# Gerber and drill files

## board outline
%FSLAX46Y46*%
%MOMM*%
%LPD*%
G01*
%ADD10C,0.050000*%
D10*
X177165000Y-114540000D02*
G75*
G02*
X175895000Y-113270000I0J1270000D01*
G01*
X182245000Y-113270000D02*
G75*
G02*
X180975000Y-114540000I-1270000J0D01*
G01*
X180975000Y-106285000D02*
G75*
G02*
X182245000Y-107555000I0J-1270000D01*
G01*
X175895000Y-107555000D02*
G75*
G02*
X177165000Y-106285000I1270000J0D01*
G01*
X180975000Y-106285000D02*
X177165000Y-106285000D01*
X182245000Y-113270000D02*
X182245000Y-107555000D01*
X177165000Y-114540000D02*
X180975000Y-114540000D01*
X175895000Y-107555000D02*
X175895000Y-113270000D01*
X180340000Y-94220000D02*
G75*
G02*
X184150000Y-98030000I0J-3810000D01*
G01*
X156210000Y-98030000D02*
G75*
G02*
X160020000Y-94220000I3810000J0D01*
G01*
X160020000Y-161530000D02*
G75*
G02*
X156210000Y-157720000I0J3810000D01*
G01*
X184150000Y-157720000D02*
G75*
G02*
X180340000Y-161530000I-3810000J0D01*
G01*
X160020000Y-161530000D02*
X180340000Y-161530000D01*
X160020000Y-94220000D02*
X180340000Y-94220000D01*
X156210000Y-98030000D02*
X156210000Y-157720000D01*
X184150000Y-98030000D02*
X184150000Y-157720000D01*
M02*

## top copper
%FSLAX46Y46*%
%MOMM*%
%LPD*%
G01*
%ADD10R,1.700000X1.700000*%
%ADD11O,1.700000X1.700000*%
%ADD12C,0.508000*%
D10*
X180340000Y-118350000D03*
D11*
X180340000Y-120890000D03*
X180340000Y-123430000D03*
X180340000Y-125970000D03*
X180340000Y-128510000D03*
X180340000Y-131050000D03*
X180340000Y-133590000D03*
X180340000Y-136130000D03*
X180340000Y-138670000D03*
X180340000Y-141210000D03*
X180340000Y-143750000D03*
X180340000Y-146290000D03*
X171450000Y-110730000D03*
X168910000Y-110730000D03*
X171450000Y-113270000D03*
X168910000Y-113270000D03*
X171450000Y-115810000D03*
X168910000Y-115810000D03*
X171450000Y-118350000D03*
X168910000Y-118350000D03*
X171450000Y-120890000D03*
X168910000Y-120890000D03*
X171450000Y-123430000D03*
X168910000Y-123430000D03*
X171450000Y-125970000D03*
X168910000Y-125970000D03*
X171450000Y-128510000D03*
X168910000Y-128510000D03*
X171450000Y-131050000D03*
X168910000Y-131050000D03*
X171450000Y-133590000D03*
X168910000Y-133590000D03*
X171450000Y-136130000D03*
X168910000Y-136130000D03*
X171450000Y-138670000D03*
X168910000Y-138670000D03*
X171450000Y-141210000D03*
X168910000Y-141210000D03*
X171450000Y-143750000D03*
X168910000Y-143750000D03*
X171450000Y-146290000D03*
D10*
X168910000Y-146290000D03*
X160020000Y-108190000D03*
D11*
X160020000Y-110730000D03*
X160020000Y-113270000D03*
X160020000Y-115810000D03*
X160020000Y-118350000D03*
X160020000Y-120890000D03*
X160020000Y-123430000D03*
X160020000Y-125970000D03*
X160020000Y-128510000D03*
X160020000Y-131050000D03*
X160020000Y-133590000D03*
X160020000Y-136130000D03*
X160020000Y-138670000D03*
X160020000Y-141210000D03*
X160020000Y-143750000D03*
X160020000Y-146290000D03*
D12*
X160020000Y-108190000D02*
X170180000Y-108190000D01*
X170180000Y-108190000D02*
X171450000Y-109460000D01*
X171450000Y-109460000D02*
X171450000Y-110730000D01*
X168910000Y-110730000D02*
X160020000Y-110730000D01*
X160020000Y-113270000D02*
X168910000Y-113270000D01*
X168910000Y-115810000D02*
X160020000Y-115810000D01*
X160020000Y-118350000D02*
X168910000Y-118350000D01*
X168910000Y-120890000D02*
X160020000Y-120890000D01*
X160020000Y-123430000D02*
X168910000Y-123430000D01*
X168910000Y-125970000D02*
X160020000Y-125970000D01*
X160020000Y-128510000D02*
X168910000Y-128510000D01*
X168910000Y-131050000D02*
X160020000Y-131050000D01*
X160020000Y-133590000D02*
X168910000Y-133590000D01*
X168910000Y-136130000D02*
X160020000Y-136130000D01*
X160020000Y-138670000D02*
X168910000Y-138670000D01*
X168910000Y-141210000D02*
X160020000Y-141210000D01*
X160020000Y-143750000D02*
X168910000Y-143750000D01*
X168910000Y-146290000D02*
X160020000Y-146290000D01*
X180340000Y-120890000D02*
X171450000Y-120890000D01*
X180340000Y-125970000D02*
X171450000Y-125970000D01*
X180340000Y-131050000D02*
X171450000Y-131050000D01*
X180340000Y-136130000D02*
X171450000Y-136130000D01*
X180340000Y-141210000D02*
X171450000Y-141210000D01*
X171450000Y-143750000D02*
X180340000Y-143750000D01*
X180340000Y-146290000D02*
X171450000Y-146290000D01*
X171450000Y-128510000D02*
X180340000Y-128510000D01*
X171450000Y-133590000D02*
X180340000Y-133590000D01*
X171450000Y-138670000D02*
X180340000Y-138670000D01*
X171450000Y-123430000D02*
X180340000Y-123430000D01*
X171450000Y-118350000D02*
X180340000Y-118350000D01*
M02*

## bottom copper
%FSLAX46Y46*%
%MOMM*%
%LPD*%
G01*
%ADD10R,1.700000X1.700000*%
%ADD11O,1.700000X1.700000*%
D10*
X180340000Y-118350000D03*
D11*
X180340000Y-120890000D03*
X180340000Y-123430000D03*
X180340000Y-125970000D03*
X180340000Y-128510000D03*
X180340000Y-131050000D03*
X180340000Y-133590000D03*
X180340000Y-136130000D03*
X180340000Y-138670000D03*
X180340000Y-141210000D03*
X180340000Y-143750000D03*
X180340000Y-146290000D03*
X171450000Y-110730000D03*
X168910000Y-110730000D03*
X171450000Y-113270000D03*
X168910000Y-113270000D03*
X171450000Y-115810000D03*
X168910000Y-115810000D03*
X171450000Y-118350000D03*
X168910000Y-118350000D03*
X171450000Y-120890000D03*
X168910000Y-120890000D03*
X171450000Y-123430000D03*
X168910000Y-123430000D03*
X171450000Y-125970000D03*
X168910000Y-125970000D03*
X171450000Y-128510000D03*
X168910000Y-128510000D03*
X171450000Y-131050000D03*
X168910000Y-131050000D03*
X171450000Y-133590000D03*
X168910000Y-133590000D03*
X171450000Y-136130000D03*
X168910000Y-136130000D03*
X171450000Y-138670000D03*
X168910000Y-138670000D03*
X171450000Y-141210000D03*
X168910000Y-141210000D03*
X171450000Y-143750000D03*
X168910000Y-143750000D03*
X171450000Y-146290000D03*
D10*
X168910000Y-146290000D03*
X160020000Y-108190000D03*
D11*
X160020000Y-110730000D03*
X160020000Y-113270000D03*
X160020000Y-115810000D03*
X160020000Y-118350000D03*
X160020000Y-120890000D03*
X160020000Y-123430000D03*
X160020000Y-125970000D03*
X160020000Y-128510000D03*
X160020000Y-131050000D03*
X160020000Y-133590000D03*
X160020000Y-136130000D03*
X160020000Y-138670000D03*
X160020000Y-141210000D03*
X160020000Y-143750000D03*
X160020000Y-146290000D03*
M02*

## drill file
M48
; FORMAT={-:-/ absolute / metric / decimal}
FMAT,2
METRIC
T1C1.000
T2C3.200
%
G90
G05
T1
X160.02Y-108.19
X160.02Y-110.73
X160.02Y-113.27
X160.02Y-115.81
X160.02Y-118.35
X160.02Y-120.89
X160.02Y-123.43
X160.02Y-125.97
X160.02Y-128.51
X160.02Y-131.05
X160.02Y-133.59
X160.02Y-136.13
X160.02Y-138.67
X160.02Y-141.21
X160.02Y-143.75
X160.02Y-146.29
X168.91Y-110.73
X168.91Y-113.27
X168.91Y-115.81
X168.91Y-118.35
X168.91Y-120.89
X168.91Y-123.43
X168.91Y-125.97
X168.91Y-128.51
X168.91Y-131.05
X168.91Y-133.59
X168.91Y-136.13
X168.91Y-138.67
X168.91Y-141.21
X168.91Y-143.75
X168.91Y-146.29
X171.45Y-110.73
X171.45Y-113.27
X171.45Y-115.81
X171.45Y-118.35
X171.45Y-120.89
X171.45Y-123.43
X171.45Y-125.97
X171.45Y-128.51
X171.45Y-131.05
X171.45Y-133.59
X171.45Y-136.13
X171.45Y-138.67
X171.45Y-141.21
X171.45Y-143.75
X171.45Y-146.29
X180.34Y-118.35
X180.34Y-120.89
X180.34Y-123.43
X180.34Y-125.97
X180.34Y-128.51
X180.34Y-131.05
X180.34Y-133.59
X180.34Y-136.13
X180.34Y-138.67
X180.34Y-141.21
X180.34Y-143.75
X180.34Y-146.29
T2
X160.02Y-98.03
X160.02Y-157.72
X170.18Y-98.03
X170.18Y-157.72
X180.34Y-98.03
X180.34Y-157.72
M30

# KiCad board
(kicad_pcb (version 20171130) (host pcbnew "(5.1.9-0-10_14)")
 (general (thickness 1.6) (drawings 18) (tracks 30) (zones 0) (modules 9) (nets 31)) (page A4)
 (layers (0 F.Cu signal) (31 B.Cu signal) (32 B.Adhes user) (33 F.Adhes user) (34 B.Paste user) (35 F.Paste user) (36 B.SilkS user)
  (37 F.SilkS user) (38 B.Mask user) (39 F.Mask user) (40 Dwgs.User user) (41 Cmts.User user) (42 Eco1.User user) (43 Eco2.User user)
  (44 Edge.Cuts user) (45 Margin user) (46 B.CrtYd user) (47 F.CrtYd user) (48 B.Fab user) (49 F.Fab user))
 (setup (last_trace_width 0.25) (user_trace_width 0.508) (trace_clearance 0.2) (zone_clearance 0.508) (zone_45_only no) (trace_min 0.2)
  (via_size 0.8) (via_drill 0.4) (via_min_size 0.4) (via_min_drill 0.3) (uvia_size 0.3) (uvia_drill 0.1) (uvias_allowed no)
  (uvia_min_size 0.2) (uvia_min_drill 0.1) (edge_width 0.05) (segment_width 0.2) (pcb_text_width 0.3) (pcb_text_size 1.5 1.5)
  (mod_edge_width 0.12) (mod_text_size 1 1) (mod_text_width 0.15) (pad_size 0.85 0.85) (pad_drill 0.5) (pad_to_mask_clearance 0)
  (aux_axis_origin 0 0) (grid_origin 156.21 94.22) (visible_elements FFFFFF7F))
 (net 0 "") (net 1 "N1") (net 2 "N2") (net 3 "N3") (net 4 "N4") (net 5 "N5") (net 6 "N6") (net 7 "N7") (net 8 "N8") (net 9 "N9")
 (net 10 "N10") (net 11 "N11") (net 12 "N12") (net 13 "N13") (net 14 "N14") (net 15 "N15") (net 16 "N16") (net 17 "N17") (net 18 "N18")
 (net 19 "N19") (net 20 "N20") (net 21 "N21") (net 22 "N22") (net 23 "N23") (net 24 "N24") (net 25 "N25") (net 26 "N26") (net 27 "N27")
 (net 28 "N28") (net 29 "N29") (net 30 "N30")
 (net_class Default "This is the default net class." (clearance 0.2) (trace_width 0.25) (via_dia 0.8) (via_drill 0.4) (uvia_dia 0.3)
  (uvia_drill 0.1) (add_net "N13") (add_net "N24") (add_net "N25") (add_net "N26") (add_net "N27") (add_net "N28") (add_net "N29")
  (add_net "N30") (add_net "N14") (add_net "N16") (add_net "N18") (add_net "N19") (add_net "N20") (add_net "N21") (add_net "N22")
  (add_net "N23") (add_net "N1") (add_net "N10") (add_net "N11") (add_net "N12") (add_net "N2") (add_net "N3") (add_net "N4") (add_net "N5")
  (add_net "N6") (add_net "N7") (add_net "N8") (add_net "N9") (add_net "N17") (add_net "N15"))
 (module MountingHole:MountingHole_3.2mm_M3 (layer F.Cu) (at 170.18 157.72)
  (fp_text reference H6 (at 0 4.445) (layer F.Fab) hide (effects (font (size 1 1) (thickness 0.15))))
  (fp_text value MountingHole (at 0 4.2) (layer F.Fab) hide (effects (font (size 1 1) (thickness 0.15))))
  (pad 1 np_thru_hole circle (at 0 0) (size 3.2 3.2) (drill 3.2) (layers *.Cu *.Mask)))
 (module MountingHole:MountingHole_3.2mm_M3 (layer F.Cu) (at 170.18 98.03)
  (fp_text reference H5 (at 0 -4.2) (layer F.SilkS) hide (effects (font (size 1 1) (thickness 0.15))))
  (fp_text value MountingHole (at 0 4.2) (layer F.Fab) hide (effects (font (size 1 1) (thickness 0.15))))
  (pad 1 np_thru_hole circle (at 0 0) (size 3.2 3.2) (drill 3.2) (layers *.Cu *.Mask)))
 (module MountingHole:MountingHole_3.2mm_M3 (layer F.Cu) (at 180.34 157.72)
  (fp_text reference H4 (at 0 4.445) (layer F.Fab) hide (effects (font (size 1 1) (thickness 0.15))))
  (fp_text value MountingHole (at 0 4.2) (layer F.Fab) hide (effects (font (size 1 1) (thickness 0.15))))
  (pad 1 np_thru_hole circle (at 0 0) (size 3.2 3.2) (drill 3.2) (layers *.Cu *.Mask)))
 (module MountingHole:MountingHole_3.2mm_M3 (layer F.Cu) (at 180.34 98.03)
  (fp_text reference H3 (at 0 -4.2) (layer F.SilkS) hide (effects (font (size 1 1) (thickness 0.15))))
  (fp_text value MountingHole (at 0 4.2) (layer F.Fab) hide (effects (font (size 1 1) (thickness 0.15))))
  (pad 1 np_thru_hole circle (at 0 0) (size 3.2 3.2) (drill 3.2) (layers *.Cu *.Mask)))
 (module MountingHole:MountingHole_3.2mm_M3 (layer F.Cu) (at 160.02 157.72)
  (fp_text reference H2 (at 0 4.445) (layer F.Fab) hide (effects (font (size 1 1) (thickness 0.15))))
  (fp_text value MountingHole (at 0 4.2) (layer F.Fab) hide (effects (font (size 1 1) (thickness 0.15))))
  (pad 1 np_thru_hole circle (at 0 0) (size 3.2 3.2) (drill 3.2) (layers *.Cu *.Mask)))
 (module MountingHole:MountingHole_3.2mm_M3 (layer F.Cu) (at 160.02 98.03)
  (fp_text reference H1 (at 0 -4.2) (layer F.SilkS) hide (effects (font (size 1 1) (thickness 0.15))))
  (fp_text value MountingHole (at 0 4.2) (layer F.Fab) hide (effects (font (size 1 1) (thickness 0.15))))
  (pad 1 np_thru_hole circle (at 0 0) (size 3.2 3.2) (drill 3.2) (layers *.Cu *.Mask)))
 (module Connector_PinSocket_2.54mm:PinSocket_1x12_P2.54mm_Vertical (layer F.Cu) (at 180.34 118.35)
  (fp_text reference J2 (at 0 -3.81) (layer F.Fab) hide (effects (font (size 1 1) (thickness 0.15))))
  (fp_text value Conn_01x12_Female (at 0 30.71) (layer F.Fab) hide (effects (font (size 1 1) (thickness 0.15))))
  (pad 1 thru_hole rect (at 0 0) (size 1.7 1.7) (drill 1) (layers *.Cu *.Mask) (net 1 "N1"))
  (pad 2 thru_hole oval (at 0 2.54) (size 1.7 1.7) (drill 1) (layers *.Cu *.Mask) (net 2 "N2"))
  (pad 3 thru_hole oval (at 0 5.08) (size 1.7 1.7) (drill 1) (layers *.Cu *.Mask) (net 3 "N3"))
  (pad 4 thru_hole oval (at 0 7.62) (size 1.7 1.7) (drill 1) (layers *.Cu *.Mask) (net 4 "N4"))
  (pad 5 thru_hole oval (at 0 10.16) (size 1.7 1.7) (drill 1) (layers *.Cu *.Mask) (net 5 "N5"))
  (pad 6 thru_hole oval (at 0 12.7) (size 1.7 1.7) (drill 1) (layers *.Cu *.Mask) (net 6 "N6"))
  (pad 7 thru_hole oval (at 0 15.24) (size 1.7 1.7) (drill 1) (layers *.Cu *.Mask) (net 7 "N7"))
  (pad 8 thru_hole oval (at 0 17.78) (size 1.7 1.7) (drill 1) (layers *.Cu *.Mask) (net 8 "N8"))
  (pad 9 thru_hole oval (at 0 20.32) (size 1.7 1.7) (drill 1) (layers *.Cu *.Mask) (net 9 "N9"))
  (pad 10 thru_hole oval (at 0 22.86) (size 1.7 1.7) (drill 1) (layers *.Cu *.Mask) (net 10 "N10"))
  (pad 11 thru_hole oval (at 0 25.4) (size 1.7 1.7) (drill 1) (layers *.Cu *.Mask) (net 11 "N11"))
  (pad 12 thru_hole oval (at 0 27.94) (size 1.7 1.7) (drill 1) (layers *.Cu *.Mask) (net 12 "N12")))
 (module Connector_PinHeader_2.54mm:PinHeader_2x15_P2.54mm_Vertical (layer B.Cu) (at 168.91 146.29)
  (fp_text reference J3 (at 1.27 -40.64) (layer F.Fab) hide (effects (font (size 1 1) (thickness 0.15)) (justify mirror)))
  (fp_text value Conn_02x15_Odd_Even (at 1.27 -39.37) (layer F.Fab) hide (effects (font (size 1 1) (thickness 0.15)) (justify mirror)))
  (pad 30 thru_hole oval (at 2.54 -35.56) (size 1.7 1.7) (drill 1) (layers *.Cu *.Mask) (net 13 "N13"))
  (pad 29 thru_hole oval (at 0 -35.56) (size 1.7 1.7) (drill 1) (layers *.Cu *.Mask) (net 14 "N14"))
  (pad 28 thru_hole oval (at 2.54 -33.02) (size 1.7 1.7) (drill 1) (layers *.Cu *.Mask) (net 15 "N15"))
  (pad 27 thru_hole oval (at 0 -33.02) (size 1.7 1.7) (drill 1) (layers *.Cu *.Mask) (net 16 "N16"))
  (pad 26 thru_hole oval (at 2.54 -30.48) (size 1.7 1.7) (drill 1) (layers *.Cu *.Mask) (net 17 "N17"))
  (pad 25 thru_hole oval (at 0 -30.48) (size 1.7 1.7) (drill 1) (layers *.Cu *.Mask) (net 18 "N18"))
  (pad 24 thru_hole oval (at 2.54 -27.94) (size 1.7 1.7) (drill 1) (layers *.Cu *.Mask) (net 1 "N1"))
  (pad 23 thru_hole oval (at 0 -27.94) (size 1.7 1.7) (drill 1) (layers *.Cu *.Mask) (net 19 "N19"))
  (pad 22 thru_hole oval (at 2.54 -25.4) (size 1.7 1.7) (drill 1) (layers *.Cu *.Mask) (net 2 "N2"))
  (pad 21 thru_hole oval (at 0 -25.4) (size 1.7 1.7) (drill 1) (layers *.Cu *.Mask) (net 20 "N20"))
  (pad 20 thru_hole oval (at 2.54 -22.86) (size 1.7 1.7) (drill 1) (layers *.Cu *.Mask) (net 3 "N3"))
  (pad 19 thru_hole oval (at 0 -22.86) (size 1.7 1.7) (drill 1) (layers *.Cu *.Mask) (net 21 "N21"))
  (pad 18 thru_hole oval (at 2.54 -20.32) (size 1.7 1.7) (drill 1) (layers *.Cu *.Mask) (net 4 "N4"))
  (pad 17 thru_hole oval (at 0 -20.32) (size 1.7 1.7) (drill 1) (layers *.Cu *.Mask) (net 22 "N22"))
  (pad 16 thru_hole oval (at 2.54 -17.78) (size 1.7 1.7) (drill 1) (layers *.Cu *.Mask) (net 5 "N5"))
  (pad 15 thru_hole oval (at 0 -17.78) (size 1.7 1.7) (drill 1) (layers *.Cu *.Mask) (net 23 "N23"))
  (pad 14 thru_hole oval (at 2.54 -15.24) (size 1.7 1.7) (drill 1) (layers *.Cu *.Mask) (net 6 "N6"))
  (pad 13 thru_hole oval (at 0 -15.24) (size 1.7 1.7) (drill 1) (layers *.Cu *.Mask) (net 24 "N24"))
  (pad 12 thru_hole oval (at 2.54 -12.7) (size 1.7 1.7) (drill 1) (layers *.Cu *.Mask) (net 7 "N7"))
  (pad 11 thru_hole oval (at 0 -12.7) (size 1.7 1.7) (drill 1) (layers *.Cu *.Mask) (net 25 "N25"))
  (pad 10 thru_hole oval (at 2.54 -10.16) (size 1.7 1.7) (drill 1) (layers *.Cu *.Mask) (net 8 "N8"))
  (pad 9 thru_hole oval (at 0 -10.16) (size 1.7 1.7) (drill 1) (layers *.Cu *.Mask) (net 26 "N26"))
  (pad 8 thru_hole oval (at 2.54 -7.62) (size 1.7 1.7) (drill 1) (layers *.Cu *.Mask) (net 9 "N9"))
  (pad 7 thru_hole oval (at 0 -7.62) (size 1.7 1.7) (drill 1) (layers *.Cu *.Mask) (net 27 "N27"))
  (pad 6 thru_hole oval (at 2.54 -5.08) (size 1.7 1.7) (drill 1) (layers *.Cu *.Mask) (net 10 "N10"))
  (pad 5 thru_hole oval (at 0 -5.08) (size 1.7 1.7) (drill 1) (layers *.Cu *.Mask) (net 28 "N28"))
  (pad 4 thru_hole oval (at 2.54 -2.54) (size 1.7 1.7) (drill 1) (layers *.Cu *.Mask) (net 11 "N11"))
  (pad 3 thru_hole oval (at 0 -2.54) (size 1.7 1.7) (drill 1) (layers *.Cu *.Mask) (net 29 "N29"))
  (pad 2 thru_hole oval (at 2.54 0) (size 1.7 1.7) (drill 1) (layers *.Cu *.Mask) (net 12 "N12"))
  (pad 1 thru_hole rect (at 0 0) (size 1.7 1.7) (drill 1) (layers *.Cu *.Mask) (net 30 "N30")))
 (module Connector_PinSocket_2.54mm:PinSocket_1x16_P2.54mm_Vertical (layer F.Cu) (at 160.02 108.19)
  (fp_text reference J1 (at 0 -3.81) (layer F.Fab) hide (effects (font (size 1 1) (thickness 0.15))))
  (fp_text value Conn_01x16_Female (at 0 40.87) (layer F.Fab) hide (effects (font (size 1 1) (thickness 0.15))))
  (pad 1 thru_hole rect (at 0 0) (size 1.7 1.7) (drill 1) (layers *.Cu *.Mask) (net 13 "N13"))
  (pad 2 thru_hole oval (at 0 2.54) (size 1.7 1.7) (drill 1) (layers *.Cu *.Mask) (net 14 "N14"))
  (pad 3 thru_hole oval (at 0 5.08) (size 1.7 1.7) (drill 1) (layers *.Cu *.Mask) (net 16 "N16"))
  (pad 4 thru_hole oval (at 0 7.62) (size 1.7 1.7) (drill 1) (layers *.Cu *.Mask) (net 18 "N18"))
  (pad 5 thru_hole oval (at 0 10.16) (size 1.7 1.7) (drill 1) (layers *.Cu *.Mask) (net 19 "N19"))
  (pad 6 thru_hole oval (at 0 12.7) (size 1.7 1.7) (drill 1) (layers *.Cu *.Mask) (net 20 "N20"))
  (pad 7 thru_hole oval (at 0 15.24) (size 1.7 1.7) (drill 1) (layers *.Cu *.Mask) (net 21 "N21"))
  (pad 8 thru_hole oval (at 0 17.78) (size 1.7 1.7) (drill 1) (layers *.Cu *.Mask) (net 22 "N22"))
  (pad 9 thru_hole oval (at 0 20.32) (size 1.7 1.7) (drill 1) (layers *.Cu *.Mask) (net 23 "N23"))
  (pad 10 thru_hole oval (at 0 22.86) (size 1.7 1.7) (drill 1) (layers *.Cu *.Mask) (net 24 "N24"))
  (pad 11 thru_hole oval (at 0 25.4) (size 1.7 1.7) (drill 1) (layers *.Cu *.Mask) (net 25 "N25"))
  (pad 12 thru_hole oval (at 0 27.94) (size 1.7 1.7) (drill 1) (layers *.Cu *.Mask) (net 26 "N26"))
  (pad 13 thru_hole oval (at 0 30.48) (size 1.7 1.7) (drill 1) (layers *.Cu *.Mask) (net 27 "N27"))
  (pad 14 thru_hole oval (at 0 33.02) (size 1.7 1.7) (drill 1) (layers *.Cu *.Mask) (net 28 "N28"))
  (pad 15 thru_hole oval (at 0 35.56) (size 1.7 1.7) (drill 1) (layers *.Cu *.Mask) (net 29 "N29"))
  (pad 16 thru_hole oval (at 0 38.1) (size 1.7 1.7) (drill 1) (layers *.Cu *.Mask) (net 30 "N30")))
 (gr_arc (start 177.165 113.27) (end 175.895 113.27) (angle -90) (layer Edge.Cuts) (width 0.05))
 (gr_arc (start 180.975 113.27) (end 180.975 114.54) (angle -90) (layer Edge.Cuts) (width 0.05))
 (gr_arc (start 180.975 107.555) (end 182.245 107.555) (angle -90) (layer Edge.Cuts) (width 0.05))
 (gr_arc (start 177.165 107.555) (end 177.165 106.285) (angle -90) (layer Edge.Cuts) (width 0.05))
 (gr_line (start 180.975 106.285) (end 177.165 106.285) (layer Edge.Cuts) (width 0.05))
 (gr_line (start 182.245 113.27) (end 182.245 107.555) (layer Edge.Cuts) (width 0.05))
 (gr_line (start 177.165 114.54) (end 180.975 114.54) (layer Edge.Cuts) (width 0.05))
 (gr_line (start 175.895 107.555) (end 175.895 113.27) (layer Edge.Cuts) (width 0.05))
 (gr_arc (start 180.34 98.03) (end 184.15 98.03) (angle -90) (layer Edge.Cuts) (width 0.05))
 (gr_arc (start 160.02 98.03) (end 160.02 94.22) (angle -90) (layer Edge.Cuts) (width 0.05))
 (gr_arc (start 160.02 157.72) (end 156.21 157.72) (angle -90) (layer Edge.Cuts) (width 0.05))
 (gr_arc (start 180.34 157.72) (end 180.34 161.53) (angle -90) (layer Edge.Cuts) (width 0.05))
 (gr_line (start 160.02 161.53) (end 180.34 161.53) (layer Edge.Cuts) (width 0.05))
 (gr_line (start 160.02 94.22) (end 180.34 94.22) (layer Edge.Cuts) (width 0.05))
 (gr_line (start 156.21 98.03) (end 156.21 157.72) (layer Edge.Cuts) (width 0.05))
 (gr_line (start 184.15 98.03) (end 184.15 157.72) (layer Edge.Cuts) (width 0.05))
 (segment (start 160.02 108.19) (end 170.18 108.19) (width 0.508) (layer F.Cu) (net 13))
 (segment (start 170.18 108.19) (end 171.45 109.46) (width 0.508) (layer F.Cu) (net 13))
 (segment (start 171.45 109.46) (end 171.45 110.73) (width 0.508) (layer F.Cu) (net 13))
 (segment (start 168.91 110.73) (end 160.02 110.73) (width 0.508) (layer F.Cu) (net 14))
 (segment (start 160.02 113.27) (end 168.91 113.27) (width 0.508) (layer F.Cu) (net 16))
 (segment (start 168.91 115.81) (end 160.02 115.81) (width 0.508) (layer F.Cu) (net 18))
 (segment (start 160.02 118.35) (end 168.91 118.35) (width 0.508) (layer F.Cu) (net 19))
 (segment (start 168.91 120.89) (end 160.02 120.89) (width 0.508) (layer F.Cu) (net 20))
 (segment (start 160.02 123.43) (end 168.91 123.43) (width 0.508) (layer F.Cu) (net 21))
 (segment (start 168.91 125.97) (end 160.02 125.97) (width 0.508) (layer F.Cu) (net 22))
 (segment (start 160.02 128.51) (end 168.91 128.51) (width 0.508) (layer F.Cu) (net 23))
 (segment (start 168.91 131.05) (end 160.02 131.05) (width 0.508) (layer F.Cu) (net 24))
 (segment (start 160.02 133.59) (end 168.91 133.59) (width 0.508) (layer F.Cu) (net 25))
 (segment (start 168.91 136.13) (end 160.02 136.13) (width 0.508) (layer F.Cu) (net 26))
 (segment (start 160.02 138.67) (end 168.91 138.67) (width 0.508) (layer F.Cu) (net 27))
 (segment (start 168.91 141.21) (end 160.02 141.21) (width 0.508) (layer F.Cu) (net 28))
 (segment (start 160.02 143.75) (end 168.91 143.75) (width 0.508) (layer F.Cu) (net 29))
 (segment (start 168.91 146.29) (end 160.02 146.29) (width 0.508) (layer F.Cu) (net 30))
 (segment (start 180.34 120.89) (end 171.45 120.89) (width 0.508) (layer F.Cu) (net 2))
 (segment (start 180.34 125.97) (end 171.45 125.97) (width 0.508) (layer F.Cu) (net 4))
 (segment (start 180.34 131.05) (end 171.45 131.05) (width 0.508) (layer F.Cu) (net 6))
 (segment (start 180.34 136.13) (end 171.45 136.13) (width 0.508) (layer F.Cu) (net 8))
 (segment (start 180.34 141.21) (end 171.45 141.21) (width 0.508) (layer F.Cu) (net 10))
 (segment (start 171.45 143.75) (end 180.34 143.75) (width 0.508) (layer F.Cu) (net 11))
 (segment (start 180.34 146.29) (end 171.45 146.29) (width 0.508) (layer F.Cu) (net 12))
 (segment (start 171.45 128.51) (end 180.34 128.51) (width 0.508) (layer F.Cu) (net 5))
 (segment (start 171.45 133.59) (end 180.34 133.59) (width 0.508) (layer F.Cu) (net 7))
 (segment (start 171.45 138.67) (end 180.34 138.67) (width 0.508) (layer F.Cu) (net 9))
 (segment (start 171.45 123.43) (end 180.34 123.43) (width 0.508) (layer F.Cu) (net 3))
 (segment (start 171.45 118.35) (end 180.34 118.35) (width 0.508) (layer F.Cu) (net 1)))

